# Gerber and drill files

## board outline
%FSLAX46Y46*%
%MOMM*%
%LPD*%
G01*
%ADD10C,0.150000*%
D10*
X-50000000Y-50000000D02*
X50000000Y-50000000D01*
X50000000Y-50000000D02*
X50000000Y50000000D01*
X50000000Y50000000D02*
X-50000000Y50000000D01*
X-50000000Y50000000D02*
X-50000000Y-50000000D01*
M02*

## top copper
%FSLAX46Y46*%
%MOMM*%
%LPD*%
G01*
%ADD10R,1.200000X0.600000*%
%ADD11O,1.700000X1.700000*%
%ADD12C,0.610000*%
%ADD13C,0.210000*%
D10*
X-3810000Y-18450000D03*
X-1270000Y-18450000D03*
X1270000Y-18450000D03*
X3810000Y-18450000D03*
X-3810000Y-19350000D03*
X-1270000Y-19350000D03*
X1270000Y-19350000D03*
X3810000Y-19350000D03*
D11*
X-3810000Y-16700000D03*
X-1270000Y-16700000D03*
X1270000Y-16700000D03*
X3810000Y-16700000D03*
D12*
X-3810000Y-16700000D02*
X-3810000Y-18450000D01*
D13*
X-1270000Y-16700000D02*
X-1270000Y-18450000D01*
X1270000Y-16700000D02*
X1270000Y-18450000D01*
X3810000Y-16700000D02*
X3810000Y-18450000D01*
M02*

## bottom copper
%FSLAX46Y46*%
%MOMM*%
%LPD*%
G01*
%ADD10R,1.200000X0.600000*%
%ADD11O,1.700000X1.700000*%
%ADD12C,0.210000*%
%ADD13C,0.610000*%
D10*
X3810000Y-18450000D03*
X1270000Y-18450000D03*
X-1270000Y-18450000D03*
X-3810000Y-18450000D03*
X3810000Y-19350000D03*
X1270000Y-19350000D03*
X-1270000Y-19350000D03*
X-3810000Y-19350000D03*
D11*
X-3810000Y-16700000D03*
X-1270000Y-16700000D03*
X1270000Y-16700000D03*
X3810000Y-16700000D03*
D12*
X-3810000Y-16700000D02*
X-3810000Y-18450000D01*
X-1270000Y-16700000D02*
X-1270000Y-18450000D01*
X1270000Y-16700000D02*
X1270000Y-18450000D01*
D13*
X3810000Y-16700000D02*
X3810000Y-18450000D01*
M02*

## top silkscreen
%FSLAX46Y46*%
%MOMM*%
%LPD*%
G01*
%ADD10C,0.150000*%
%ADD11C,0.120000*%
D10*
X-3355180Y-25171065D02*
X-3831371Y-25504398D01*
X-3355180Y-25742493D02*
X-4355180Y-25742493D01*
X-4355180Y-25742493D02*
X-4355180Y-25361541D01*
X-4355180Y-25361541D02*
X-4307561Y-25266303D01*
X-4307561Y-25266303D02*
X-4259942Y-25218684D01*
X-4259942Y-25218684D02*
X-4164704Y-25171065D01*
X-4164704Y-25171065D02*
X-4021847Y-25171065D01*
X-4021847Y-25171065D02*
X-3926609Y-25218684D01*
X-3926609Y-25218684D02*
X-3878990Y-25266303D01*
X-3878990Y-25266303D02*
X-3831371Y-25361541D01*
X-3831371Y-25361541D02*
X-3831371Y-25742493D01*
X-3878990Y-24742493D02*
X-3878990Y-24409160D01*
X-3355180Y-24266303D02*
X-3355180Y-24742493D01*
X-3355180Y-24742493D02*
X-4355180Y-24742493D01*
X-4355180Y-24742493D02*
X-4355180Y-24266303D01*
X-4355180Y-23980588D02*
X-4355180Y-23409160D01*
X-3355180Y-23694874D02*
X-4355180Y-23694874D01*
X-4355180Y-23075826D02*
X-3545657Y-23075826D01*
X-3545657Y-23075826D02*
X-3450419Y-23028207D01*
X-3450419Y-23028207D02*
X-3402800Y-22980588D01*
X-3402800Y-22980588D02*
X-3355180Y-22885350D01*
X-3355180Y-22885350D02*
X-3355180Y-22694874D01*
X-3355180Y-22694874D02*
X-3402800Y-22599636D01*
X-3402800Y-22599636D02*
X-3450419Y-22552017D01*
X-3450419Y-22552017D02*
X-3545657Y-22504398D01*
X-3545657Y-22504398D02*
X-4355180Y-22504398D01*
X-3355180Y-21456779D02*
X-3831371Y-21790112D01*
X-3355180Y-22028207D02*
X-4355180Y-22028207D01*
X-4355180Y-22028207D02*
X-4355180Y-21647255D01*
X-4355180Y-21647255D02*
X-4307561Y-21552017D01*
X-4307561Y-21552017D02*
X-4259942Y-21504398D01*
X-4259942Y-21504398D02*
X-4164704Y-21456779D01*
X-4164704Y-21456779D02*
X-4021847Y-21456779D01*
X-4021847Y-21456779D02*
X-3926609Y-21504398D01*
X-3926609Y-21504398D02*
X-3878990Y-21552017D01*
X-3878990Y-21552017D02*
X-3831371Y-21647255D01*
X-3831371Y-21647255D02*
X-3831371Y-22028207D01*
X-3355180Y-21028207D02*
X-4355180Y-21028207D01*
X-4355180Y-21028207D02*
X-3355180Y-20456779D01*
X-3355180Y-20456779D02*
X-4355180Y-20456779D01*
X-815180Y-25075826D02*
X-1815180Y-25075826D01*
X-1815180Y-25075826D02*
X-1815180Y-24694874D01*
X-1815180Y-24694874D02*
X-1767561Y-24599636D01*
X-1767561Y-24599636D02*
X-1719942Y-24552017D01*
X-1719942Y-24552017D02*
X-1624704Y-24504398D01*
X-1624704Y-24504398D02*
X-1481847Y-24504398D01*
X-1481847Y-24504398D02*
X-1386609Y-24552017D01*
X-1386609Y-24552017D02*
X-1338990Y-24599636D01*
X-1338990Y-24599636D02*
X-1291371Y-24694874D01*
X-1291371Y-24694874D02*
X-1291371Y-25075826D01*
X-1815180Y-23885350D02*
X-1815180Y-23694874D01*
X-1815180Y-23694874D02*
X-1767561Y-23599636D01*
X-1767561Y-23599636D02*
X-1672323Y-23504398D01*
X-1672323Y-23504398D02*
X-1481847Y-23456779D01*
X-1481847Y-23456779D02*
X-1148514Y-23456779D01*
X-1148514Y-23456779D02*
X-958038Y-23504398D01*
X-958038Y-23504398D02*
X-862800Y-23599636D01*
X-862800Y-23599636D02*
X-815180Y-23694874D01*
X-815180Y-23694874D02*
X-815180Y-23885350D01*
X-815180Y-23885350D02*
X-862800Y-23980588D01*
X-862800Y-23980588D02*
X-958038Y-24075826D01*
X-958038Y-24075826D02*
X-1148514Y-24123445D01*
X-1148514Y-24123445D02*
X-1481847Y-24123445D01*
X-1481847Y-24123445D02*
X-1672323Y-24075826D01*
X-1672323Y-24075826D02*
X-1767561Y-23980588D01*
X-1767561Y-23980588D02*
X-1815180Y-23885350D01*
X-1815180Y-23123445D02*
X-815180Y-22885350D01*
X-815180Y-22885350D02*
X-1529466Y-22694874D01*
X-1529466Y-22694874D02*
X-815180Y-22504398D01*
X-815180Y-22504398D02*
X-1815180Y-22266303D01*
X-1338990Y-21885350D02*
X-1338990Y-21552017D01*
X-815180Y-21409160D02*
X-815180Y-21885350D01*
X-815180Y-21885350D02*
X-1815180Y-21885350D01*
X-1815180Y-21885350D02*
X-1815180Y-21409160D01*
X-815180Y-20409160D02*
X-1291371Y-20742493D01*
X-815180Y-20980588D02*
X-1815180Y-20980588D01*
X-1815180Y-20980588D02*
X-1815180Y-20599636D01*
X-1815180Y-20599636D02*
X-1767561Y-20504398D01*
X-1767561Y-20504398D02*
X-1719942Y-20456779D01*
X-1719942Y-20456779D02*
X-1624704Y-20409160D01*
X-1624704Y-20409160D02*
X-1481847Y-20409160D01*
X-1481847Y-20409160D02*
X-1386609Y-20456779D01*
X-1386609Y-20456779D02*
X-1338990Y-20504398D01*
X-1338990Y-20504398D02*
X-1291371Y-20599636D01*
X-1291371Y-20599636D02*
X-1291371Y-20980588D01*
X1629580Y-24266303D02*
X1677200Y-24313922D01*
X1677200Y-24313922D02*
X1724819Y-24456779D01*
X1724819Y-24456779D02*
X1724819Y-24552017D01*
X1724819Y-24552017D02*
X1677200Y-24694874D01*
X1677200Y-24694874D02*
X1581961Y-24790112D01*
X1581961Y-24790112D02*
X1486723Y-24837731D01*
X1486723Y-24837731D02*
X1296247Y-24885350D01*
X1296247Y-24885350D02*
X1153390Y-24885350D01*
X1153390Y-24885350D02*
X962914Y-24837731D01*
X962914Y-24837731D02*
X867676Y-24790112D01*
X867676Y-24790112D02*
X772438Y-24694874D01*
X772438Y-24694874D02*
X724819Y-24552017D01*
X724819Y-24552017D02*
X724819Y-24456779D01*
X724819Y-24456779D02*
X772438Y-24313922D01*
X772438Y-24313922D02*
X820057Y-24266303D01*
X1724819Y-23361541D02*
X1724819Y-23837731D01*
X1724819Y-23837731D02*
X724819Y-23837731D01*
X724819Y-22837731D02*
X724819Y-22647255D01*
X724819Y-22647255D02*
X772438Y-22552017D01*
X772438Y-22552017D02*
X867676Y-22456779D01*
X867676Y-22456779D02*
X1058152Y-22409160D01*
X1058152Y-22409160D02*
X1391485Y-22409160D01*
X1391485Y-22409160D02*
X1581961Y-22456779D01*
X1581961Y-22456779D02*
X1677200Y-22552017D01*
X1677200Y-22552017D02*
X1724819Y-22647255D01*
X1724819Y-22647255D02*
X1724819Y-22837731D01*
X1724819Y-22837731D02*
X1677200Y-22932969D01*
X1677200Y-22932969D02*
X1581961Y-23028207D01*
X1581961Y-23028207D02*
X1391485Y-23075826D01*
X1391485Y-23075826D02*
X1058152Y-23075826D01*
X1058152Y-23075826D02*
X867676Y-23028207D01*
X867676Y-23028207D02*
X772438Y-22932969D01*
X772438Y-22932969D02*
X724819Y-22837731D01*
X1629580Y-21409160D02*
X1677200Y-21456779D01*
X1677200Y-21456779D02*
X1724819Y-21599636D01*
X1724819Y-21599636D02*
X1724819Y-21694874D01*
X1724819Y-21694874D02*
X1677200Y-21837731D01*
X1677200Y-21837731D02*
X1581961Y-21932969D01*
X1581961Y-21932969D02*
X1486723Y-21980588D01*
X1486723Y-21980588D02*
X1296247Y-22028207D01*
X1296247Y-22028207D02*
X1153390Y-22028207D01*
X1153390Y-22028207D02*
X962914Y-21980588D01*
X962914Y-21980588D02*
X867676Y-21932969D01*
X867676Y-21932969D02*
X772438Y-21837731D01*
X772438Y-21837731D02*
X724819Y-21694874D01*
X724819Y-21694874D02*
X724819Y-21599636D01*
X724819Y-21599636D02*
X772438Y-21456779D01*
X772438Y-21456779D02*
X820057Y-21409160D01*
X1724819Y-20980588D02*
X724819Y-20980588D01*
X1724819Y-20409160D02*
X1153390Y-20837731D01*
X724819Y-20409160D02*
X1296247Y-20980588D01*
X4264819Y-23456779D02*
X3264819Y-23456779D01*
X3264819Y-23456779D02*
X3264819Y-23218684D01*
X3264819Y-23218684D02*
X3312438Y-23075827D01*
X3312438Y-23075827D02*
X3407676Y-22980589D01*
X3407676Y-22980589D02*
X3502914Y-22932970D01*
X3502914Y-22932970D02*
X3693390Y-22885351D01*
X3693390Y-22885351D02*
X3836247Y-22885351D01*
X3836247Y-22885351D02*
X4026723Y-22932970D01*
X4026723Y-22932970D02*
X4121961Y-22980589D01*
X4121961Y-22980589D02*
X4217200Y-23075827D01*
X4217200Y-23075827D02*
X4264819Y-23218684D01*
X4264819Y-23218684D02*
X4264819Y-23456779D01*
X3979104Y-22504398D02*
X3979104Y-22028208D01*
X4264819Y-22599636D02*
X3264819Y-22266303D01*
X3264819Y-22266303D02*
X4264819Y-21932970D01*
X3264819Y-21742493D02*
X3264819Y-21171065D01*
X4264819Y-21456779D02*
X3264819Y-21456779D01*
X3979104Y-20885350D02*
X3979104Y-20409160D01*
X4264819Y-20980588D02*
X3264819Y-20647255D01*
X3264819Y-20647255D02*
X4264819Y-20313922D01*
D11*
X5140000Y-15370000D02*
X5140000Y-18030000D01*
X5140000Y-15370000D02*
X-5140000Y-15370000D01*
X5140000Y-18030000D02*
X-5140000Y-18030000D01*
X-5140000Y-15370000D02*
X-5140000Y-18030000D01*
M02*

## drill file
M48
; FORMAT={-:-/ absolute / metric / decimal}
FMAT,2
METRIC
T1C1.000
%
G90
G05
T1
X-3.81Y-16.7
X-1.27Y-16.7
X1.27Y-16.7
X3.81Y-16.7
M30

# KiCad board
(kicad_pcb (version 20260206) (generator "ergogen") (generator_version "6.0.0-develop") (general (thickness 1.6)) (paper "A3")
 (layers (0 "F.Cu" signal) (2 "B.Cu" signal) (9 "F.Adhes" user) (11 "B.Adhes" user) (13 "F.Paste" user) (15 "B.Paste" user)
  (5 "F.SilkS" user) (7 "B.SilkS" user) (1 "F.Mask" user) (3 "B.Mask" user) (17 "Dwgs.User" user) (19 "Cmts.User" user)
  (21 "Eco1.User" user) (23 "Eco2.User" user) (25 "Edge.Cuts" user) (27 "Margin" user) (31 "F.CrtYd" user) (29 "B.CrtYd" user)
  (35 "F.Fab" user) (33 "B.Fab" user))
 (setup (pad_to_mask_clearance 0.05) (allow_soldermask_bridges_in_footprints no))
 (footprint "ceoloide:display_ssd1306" (layer "B.Cu") (at 0 0 0)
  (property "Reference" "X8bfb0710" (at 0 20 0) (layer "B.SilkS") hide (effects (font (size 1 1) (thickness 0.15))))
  (fp_line (start 5.14 15.37) (end 5.14 18.03) (layer "F.SilkS") (stroke (width 0.12) (type solid)))
  (fp_line (start 5.14 15.37) (end -5.14 15.37) (layer "F.SilkS") (stroke (width 0.12) (type solid)))
  (fp_line (start 5.14 18.03) (end -5.14 18.03) (layer "F.SilkS") (stroke (width 0.12) (type solid)))
  (fp_line (start -5.14 15.37) (end -5.14 18.03) (layer "F.SilkS") (stroke (width 0.12) (type solid)))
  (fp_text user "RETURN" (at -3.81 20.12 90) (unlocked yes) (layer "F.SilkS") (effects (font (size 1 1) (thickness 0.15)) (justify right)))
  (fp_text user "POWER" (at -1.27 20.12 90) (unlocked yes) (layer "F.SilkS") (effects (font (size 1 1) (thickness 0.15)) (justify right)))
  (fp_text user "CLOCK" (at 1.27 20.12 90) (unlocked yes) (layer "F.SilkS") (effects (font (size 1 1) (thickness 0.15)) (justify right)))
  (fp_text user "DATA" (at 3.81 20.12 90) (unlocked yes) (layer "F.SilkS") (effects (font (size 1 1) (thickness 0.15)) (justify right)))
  (pad "14" smd rect (at -3.81 18.450000000000003 90) (size 0.6 1.2) (layers "F.Cu" "F.Paste" "F.Mask") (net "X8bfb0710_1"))
  (pad "15" smd rect (at -1.27 18.450000000000003 90) (size 0.6 1.2) (layers "F.Cu" "F.Paste" "F.Mask") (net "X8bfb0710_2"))
  (pad "16" smd rect (at 1.27 18.450000000000003 90) (size 0.6 1.2) (layers "F.Cu" "F.Paste" "F.Mask") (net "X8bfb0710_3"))
  (pad "17" smd rect (at 3.81 18.450000000000003 90) (size 0.6 1.2) (layers "F.Cu" "F.Paste" "F.Mask") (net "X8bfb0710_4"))
  (pad "10" smd rect (at -3.81 19.35 90) (size 0.6 1.2) (layers "F.Cu" "F.Paste" "F.Mask") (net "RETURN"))
  (pad "11" smd rect (at -1.27 19.35 90) (size 0.6 1.2) (layers "F.Cu" "F.Paste" "F.Mask") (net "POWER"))
  (pad "12" smd rect (at 1.27 19.35 90) (size 0.6 1.2) (layers "F.Cu" "F.Paste" "F.Mask") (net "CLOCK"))
  (pad "13" smd rect (at 3.81 19.35 90) (size 0.6 1.2) (layers "F.Cu" "F.Paste" "F.Mask") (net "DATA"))
  (pad "24" smd rect (at 3.81 18.450000000000003 270) (size 0.6 1.2) (layers "B.Cu" "B.Paste" "B.Mask") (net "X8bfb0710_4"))
  (pad "25" smd rect (at 1.27 18.450000000000003 270) (size 0.6 1.2) (layers "B.Cu" "B.Paste" "B.Mask") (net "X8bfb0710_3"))
  (pad "26" smd rect (at -1.27 18.450000000000003 270) (size 0.6 1.2) (layers "B.Cu" "B.Paste" "B.Mask") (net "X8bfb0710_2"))
  (pad "27" smd rect (at -3.81 18.450000000000003 270) (size 0.6 1.2) (layers "B.Cu" "B.Paste" "B.Mask") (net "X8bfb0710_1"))
  (pad "20" smd rect (at 3.81 19.35 270) (size 0.6 1.2) (layers "B.Cu" "B.Paste" "B.Mask") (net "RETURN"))
  (pad "21" smd rect (at 1.27 19.35 270) (size 0.6 1.2) (layers "B.Cu" "B.Paste" "B.Mask") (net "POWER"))
  (pad "22" smd rect (at -1.27 19.35 270) (size 0.6 1.2) (layers "B.Cu" "B.Paste" "B.Mask") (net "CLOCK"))
  (pad "23" smd rect (at -3.81 19.35 270) (size 0.6 1.2) (layers "B.Cu" "B.Paste" "B.Mask") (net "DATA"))
  (pad "1" thru_hole oval (at -3.81 16.7 270) (size 1.7 1.7) (drill 1) (layers "*.Cu" "*.Mask") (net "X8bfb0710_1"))
  (pad "2" thru_hole oval (at -1.27 16.7 270) (size 1.7 1.7) (drill 1) (layers "*.Cu" "*.Mask") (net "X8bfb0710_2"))
  (pad "3" thru_hole oval (at 1.27 16.7 270) (size 1.7 1.7) (drill 1) (layers "*.Cu" "*.Mask") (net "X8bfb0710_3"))
  (pad "4" thru_hole oval (at 3.81 16.7 270) (size 1.7 1.7) (drill 1) (layers "*.Cu" "*.Mask") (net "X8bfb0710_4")))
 (segment (start -3.81 16.7) (end -3.81 18.45) (width 0.61) (layer "F.Cu") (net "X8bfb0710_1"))
 (segment (start -1.27 16.7) (end -1.27 18.45) (width 0.21) (layer "F.Cu") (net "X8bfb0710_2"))
 (segment (start 1.27 16.7) (end 1.27 18.45) (width 0.21) (layer "F.Cu") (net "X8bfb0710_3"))
 (segment (start 3.81 16.7) (end 3.81 18.45) (width 0.21) (layer "F.Cu") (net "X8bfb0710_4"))
 (segment (start -3.81 16.7) (end -3.81 18.45) (width 0.21) (layer "B.Cu") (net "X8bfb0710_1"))
 (segment (start -1.27 16.7) (end -1.27 18.45) (width 0.21) (layer "B.Cu") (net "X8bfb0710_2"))
 (segment (start 1.27 16.7) (end 1.27 18.45) (width 0.21) (layer "B.Cu") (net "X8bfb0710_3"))
 (segment (start 3.81 16.7) (end 3.81 18.45) (width 0.61) (layer "B.Cu") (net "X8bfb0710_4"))
 (gr_line (start -50 50) (end 50 50) (layer Edge.Cuts) (stroke (width 0.15) (type default)))
 (gr_line (start 50 50) (end 50 -50) (layer Edge.Cuts) (stroke (width 0.15) (type default)))
 (gr_line (start 50 -50) (end -50 -50) (layer Edge.Cuts) (stroke (width 0.15) (type default)))
 (gr_line (start -50 -50) (end -50 50) (layer Edge.Cuts) (stroke (width 0.15) (type default))))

